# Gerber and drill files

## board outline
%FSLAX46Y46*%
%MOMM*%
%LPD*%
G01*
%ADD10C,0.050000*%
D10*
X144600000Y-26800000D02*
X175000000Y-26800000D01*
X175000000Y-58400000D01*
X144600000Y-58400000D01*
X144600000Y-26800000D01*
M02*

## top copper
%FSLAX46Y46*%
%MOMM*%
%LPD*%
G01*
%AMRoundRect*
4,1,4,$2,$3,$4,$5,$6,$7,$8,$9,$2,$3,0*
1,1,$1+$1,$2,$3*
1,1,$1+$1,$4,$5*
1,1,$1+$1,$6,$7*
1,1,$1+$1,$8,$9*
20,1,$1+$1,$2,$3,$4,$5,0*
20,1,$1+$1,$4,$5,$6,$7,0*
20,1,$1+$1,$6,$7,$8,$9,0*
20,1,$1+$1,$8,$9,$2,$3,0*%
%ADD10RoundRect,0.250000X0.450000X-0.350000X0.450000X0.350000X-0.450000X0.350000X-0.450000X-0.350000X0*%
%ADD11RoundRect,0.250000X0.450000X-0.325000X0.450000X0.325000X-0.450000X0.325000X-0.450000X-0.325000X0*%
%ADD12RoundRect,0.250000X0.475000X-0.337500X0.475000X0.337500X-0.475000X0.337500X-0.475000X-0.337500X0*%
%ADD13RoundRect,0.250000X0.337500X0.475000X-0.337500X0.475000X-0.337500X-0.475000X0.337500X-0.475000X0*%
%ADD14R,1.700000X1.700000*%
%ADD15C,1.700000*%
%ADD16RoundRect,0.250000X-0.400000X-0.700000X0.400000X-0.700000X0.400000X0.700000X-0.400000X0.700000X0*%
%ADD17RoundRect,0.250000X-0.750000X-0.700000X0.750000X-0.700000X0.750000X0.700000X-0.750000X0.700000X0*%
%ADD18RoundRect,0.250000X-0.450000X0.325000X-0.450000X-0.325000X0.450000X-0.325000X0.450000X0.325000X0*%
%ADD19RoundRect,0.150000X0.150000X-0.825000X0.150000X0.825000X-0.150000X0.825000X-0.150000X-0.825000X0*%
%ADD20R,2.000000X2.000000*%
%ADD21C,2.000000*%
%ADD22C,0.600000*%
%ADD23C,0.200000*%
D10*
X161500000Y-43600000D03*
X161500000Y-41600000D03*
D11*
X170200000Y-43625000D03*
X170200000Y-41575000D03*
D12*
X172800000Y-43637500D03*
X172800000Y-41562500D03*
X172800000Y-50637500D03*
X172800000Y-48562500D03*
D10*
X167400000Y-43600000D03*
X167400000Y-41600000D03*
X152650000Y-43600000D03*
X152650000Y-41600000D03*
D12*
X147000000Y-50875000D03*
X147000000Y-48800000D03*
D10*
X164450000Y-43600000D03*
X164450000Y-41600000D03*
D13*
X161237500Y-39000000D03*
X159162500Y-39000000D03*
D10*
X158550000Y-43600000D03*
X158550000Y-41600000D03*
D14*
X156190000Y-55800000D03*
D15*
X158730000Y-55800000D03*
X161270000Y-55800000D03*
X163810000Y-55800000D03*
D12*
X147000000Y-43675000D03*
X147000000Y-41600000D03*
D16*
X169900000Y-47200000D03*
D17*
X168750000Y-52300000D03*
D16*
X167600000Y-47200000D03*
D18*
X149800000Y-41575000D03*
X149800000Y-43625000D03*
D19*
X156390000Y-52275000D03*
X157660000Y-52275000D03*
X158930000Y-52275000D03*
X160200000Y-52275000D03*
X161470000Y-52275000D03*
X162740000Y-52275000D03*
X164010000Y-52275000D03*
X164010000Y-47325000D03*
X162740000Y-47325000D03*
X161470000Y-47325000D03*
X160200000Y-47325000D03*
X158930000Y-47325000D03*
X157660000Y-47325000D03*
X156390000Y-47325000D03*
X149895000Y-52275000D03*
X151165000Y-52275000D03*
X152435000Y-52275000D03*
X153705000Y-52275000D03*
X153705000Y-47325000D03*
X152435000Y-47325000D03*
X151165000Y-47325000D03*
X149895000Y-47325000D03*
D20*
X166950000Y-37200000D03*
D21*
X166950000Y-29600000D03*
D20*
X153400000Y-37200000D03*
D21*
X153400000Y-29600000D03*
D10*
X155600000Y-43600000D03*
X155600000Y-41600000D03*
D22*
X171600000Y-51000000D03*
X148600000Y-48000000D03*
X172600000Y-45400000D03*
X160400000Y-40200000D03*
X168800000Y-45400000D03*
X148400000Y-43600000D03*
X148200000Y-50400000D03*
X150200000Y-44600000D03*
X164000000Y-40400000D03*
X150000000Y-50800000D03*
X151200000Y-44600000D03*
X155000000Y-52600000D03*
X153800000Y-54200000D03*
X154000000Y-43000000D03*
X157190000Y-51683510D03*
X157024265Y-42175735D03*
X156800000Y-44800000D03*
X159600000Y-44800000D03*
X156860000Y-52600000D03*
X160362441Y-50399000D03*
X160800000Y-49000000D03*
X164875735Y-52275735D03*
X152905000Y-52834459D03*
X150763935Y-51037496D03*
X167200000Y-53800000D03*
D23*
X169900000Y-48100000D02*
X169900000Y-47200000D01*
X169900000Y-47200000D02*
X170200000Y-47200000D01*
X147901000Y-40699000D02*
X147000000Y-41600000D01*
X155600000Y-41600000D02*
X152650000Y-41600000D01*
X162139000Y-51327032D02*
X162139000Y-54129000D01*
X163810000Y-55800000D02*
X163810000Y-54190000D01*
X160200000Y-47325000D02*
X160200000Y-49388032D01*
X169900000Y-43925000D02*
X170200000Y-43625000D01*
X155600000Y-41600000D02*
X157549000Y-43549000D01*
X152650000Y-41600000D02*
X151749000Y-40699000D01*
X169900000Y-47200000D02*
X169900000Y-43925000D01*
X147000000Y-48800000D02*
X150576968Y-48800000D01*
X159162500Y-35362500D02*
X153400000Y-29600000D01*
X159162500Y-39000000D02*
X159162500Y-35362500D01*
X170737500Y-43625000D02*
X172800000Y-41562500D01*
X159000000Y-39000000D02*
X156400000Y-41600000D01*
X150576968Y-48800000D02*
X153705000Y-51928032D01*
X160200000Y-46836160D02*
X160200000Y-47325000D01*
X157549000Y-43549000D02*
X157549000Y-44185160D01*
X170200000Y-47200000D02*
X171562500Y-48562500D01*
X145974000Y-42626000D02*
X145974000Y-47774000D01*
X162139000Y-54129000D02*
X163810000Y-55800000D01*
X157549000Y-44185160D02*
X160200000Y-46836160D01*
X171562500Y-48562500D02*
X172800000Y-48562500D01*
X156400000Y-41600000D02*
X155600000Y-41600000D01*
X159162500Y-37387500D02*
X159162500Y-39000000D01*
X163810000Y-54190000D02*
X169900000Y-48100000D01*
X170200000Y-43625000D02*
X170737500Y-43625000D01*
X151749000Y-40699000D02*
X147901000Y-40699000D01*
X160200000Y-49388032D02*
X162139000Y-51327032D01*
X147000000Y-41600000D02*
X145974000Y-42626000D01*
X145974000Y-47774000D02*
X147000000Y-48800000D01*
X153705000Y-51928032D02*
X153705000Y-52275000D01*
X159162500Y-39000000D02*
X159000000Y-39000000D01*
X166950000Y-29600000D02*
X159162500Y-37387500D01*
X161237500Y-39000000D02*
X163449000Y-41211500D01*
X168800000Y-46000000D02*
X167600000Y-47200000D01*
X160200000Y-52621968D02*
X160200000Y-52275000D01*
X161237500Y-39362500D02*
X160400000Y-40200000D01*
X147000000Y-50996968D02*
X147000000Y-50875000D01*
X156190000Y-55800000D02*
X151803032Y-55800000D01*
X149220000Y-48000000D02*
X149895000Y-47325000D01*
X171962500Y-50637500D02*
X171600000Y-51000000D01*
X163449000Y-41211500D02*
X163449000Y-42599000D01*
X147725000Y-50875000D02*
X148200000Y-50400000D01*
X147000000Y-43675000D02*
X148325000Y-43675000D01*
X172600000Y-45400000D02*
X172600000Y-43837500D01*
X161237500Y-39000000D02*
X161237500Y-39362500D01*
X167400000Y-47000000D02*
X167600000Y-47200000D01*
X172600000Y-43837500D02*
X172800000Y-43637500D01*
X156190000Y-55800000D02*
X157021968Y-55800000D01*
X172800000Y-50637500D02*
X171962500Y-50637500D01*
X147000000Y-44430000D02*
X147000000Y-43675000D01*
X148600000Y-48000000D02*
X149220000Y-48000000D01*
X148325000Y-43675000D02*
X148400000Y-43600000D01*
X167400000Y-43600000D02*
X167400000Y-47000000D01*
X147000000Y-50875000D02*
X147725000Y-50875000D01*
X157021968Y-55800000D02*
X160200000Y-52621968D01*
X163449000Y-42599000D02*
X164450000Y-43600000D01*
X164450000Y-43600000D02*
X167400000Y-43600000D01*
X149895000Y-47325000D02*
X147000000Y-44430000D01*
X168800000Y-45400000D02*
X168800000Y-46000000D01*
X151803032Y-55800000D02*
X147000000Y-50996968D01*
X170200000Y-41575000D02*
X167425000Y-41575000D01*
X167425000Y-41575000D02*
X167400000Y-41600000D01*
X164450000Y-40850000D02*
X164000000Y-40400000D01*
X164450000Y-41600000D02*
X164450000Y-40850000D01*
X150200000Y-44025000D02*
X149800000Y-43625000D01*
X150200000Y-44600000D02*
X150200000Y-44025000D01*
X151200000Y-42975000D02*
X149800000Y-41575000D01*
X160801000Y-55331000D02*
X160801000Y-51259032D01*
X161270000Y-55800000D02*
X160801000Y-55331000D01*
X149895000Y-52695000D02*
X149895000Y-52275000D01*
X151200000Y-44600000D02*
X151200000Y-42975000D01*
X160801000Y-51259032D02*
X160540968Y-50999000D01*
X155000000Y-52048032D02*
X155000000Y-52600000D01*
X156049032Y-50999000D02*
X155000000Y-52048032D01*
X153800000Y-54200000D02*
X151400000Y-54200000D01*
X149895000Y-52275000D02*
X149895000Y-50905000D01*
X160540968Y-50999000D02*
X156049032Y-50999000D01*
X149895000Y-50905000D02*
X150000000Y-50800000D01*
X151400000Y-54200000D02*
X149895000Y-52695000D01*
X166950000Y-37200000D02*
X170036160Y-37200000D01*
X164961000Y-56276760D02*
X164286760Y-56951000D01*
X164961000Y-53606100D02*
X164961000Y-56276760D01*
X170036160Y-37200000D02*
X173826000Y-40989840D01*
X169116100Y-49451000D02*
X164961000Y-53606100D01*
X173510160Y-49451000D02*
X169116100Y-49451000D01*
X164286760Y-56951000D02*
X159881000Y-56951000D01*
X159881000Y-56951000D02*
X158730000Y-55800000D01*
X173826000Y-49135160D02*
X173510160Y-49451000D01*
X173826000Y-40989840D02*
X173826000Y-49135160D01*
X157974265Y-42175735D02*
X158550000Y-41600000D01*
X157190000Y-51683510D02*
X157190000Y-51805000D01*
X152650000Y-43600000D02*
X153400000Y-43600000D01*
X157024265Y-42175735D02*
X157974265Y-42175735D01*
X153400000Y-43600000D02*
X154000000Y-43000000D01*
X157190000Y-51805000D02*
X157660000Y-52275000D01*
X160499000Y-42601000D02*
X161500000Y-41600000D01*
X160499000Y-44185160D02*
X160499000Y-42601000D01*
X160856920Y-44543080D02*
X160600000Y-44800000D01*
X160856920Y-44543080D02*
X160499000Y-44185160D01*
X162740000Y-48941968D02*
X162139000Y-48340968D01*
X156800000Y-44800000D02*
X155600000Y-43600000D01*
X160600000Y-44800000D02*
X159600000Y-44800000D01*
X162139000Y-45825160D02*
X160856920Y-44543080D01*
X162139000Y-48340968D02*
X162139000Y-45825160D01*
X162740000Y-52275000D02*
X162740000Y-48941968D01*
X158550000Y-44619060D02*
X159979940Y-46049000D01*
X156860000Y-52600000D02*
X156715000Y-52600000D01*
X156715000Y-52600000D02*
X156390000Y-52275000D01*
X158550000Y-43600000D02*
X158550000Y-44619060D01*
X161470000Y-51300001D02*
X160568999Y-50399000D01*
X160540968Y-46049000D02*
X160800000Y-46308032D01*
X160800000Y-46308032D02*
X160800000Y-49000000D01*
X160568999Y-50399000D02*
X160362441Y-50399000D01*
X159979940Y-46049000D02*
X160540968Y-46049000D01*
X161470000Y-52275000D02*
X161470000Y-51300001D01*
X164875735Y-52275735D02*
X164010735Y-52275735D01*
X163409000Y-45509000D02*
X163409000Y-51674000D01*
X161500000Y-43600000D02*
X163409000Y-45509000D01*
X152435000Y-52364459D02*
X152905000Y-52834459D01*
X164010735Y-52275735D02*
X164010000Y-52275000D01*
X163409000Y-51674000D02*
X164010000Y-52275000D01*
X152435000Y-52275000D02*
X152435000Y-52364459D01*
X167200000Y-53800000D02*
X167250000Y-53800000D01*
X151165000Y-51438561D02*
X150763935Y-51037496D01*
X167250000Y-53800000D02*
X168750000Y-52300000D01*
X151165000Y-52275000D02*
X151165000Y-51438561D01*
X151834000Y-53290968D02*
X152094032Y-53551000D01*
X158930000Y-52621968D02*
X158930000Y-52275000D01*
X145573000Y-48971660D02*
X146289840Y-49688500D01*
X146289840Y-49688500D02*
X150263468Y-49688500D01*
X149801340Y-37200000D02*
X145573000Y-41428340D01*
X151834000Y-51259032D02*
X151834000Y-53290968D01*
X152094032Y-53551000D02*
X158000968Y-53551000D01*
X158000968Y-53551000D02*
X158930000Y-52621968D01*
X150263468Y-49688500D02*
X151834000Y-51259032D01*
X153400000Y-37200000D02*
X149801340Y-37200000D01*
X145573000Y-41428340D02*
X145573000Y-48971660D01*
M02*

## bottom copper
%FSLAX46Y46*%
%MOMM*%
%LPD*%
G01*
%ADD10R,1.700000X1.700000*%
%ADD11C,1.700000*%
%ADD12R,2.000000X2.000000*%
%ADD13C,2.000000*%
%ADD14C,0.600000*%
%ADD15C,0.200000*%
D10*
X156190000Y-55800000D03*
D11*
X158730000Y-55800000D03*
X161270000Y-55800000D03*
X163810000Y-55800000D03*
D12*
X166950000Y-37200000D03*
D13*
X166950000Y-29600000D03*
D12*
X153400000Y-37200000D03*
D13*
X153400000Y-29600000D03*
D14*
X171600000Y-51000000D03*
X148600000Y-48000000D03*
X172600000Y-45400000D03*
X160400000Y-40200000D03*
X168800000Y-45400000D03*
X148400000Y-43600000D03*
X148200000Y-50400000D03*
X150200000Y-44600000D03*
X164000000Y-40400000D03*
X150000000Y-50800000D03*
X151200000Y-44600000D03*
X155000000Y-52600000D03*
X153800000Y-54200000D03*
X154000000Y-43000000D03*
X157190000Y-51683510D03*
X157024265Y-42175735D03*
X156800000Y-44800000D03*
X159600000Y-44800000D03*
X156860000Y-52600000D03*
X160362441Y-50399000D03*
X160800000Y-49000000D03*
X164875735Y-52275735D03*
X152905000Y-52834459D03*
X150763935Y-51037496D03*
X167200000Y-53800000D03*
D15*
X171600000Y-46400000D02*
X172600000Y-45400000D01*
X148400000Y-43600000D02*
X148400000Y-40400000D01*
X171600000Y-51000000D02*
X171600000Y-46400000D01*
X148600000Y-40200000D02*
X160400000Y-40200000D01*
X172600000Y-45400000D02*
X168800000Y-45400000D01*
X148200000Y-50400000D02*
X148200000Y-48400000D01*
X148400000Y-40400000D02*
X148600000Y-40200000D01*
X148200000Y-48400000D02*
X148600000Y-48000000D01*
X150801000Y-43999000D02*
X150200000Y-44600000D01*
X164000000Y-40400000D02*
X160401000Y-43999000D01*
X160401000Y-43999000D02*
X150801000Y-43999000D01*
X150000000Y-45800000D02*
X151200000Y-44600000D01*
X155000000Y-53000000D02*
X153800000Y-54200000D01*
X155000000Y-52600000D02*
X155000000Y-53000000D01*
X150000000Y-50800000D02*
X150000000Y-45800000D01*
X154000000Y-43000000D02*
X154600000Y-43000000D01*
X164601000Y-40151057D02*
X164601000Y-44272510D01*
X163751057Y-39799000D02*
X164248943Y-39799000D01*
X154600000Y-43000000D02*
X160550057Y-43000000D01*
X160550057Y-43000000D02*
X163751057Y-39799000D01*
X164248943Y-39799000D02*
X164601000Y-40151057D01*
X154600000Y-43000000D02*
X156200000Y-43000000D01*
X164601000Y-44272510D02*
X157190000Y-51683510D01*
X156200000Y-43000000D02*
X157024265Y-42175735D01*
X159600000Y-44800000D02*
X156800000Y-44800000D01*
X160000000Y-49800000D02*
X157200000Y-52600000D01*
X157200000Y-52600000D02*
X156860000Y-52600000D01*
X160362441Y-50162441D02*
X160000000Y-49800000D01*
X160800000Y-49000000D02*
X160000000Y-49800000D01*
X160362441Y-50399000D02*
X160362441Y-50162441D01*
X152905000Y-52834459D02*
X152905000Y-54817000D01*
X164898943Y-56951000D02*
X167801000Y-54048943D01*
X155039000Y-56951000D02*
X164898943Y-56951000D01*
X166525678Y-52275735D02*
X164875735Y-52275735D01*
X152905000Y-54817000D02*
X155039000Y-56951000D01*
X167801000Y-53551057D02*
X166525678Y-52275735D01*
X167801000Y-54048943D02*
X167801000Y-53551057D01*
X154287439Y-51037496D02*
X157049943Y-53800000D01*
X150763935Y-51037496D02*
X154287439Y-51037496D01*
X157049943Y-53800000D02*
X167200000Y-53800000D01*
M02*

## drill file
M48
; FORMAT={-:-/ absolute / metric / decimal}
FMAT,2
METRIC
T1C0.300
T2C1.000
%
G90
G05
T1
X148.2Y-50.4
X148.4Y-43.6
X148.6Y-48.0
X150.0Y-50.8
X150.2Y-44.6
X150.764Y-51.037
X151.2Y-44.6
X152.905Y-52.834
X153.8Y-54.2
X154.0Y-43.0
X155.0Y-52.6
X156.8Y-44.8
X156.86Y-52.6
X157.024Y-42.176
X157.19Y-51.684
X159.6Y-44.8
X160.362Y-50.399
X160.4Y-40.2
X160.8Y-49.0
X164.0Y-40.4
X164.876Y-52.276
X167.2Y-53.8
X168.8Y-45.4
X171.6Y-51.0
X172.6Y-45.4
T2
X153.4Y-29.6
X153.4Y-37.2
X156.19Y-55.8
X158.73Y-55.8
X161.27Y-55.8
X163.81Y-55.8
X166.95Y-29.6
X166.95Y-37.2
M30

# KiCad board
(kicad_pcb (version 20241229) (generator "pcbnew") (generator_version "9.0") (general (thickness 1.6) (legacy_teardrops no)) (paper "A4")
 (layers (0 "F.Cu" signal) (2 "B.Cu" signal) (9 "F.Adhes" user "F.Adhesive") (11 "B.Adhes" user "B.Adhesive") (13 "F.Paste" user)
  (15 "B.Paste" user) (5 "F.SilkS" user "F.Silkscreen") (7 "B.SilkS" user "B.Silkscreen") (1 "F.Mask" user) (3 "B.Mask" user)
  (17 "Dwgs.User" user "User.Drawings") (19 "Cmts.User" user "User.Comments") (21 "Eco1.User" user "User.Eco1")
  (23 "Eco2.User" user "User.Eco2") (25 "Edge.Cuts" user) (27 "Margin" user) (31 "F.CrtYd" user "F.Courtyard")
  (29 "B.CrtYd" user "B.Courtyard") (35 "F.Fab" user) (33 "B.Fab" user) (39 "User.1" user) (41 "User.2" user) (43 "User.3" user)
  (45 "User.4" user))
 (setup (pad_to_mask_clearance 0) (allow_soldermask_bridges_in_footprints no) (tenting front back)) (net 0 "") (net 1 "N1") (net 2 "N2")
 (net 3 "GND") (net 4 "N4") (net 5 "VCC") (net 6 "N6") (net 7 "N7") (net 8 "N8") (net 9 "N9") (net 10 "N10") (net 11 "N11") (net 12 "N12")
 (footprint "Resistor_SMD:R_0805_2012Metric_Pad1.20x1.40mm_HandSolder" (layer "F.Cu") (at 161.5 42.6 90)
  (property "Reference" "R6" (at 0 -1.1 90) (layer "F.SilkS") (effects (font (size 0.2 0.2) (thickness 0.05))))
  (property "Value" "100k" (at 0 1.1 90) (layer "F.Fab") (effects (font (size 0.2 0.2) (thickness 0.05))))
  (pad "1" smd roundrect (at -1 0 90) (size 1.2 1.4) (layers "F.Cu" "F.Mask" "F.Paste") (roundrect_rratio 0.208333) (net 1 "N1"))
  (pad "2" smd roundrect (at 1 0 90) (size 1.2 1.4) (layers "F.Cu" "F.Mask" "F.Paste") (roundrect_rratio 0.208333) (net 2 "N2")))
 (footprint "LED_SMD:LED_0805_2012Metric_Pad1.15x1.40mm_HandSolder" (layer "F.Cu") (at 170.2 42.6 90)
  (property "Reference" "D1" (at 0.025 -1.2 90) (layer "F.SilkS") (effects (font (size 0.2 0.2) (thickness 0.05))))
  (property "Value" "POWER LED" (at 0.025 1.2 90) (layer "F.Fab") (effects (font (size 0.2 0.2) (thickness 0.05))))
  (pad "1" smd roundrect (at -1.025 0 90) (size 1.15 1.4) (layers "F.Cu" "F.Mask" "F.Paste") (roundrect_rratio 0.217391) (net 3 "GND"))
  (pad "2" smd roundrect (at 1.025 0 90) (size 1.15 1.4) (layers "F.Cu" "F.Mask" "F.Paste") (roundrect_rratio 0.217391) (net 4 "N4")))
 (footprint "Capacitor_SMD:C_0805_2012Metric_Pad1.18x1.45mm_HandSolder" (layer "F.Cu") (at 172.8 42.6 90)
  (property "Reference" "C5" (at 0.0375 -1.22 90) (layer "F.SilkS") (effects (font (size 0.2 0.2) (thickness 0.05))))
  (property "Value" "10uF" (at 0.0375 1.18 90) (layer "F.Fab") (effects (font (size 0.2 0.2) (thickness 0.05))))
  (pad "1" smd roundrect (at -1.0375 0 90) (size 1.175 1.45) (layers "F.Cu" "F.Mask" "F.Paste") (roundrect_rratio 0.212766) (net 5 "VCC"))
  (pad "2" smd roundrect (at 1.0375 0 90) (size 1.175 1.45) (layers "F.Cu" "F.Mask" "F.Paste") (roundrect_rratio 0.212766) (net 3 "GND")))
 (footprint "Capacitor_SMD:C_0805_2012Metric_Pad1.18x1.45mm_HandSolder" (layer "F.Cu") (at 172.8 49.6 90)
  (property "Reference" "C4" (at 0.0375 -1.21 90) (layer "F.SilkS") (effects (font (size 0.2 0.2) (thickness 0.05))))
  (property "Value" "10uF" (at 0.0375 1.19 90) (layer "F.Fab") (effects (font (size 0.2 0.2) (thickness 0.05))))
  (pad "1" smd roundrect (at -1.0375 0 90) (size 1.175 1.45) (layers "F.Cu" "F.Mask" "F.Paste") (roundrect_rratio 0.212766) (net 5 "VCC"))
  (pad "2" smd roundrect (at 1.0375 0 90) (size 1.175 1.45) (layers "F.Cu" "F.Mask" "F.Paste") (roundrect_rratio 0.212766) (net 3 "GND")))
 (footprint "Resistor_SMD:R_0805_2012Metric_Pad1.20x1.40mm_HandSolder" (layer "F.Cu") (at 167.4 42.6 90)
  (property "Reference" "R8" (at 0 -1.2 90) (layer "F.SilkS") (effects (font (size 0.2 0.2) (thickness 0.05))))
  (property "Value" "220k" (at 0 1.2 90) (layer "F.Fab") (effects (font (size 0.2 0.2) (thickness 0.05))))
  (pad "1" smd roundrect (at -1 0 90) (size 1.2 1.4) (layers "F.Cu" "F.Mask" "F.Paste") (roundrect_rratio 0.208333) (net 5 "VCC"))
  (pad "2" smd roundrect (at 1 0 90) (size 1.2 1.4) (layers "F.Cu" "F.Mask" "F.Paste") (roundrect_rratio 0.208333) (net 4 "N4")))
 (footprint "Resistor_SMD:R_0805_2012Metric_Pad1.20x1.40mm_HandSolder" (layer "F.Cu") (at 152.65 42.6 90)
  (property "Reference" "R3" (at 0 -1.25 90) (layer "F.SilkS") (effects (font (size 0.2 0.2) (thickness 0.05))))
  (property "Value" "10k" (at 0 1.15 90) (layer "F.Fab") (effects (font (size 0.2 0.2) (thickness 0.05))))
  (pad "1" smd roundrect (at -1 0 90) (size 1.2 1.4) (layers "F.Cu" "F.Mask" "F.Paste") (roundrect_rratio 0.208333) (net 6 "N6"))
  (pad "2" smd roundrect (at 1 0 90) (size 1.2 1.4) (layers "F.Cu" "F.Mask" "F.Paste") (roundrect_rratio 0.208333) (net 3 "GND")))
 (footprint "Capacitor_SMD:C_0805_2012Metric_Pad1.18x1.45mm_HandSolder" (layer "F.Cu") (at 147 49.8375 90)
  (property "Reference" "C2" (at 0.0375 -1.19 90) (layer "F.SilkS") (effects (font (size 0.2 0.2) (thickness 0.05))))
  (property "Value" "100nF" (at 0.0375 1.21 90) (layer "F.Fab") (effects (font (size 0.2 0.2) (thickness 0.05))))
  (pad "1" smd roundrect (at -1.0375 0 90) (size 1.175 1.45) (layers "F.Cu" "F.Mask" "F.Paste") (roundrect_rratio 0.212766) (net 5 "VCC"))
  (pad "2" smd roundrect (at 1.0375 0 90) (size 1.175 1.45) (layers "F.Cu" "F.Mask" "F.Paste") (roundrect_rratio 0.212766) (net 3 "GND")))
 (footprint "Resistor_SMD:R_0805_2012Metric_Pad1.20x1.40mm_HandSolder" (layer "F.Cu") (at 164.45 42.6 90)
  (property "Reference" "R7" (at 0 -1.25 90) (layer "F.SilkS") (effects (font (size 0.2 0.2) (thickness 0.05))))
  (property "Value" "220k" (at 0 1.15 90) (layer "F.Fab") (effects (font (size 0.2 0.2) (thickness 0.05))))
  (pad "1" smd roundrect (at -1 0 90) (size 1.2 1.4) (layers "F.Cu" "F.Mask" "F.Paste") (roundrect_rratio 0.208333) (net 5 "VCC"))
  (pad "2" smd roundrect (at 1 0 90) (size 1.2 1.4) (layers "F.Cu" "F.Mask" "F.Paste") (roundrect_rratio 0.208333) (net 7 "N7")))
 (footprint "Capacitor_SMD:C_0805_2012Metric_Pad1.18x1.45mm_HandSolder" (layer "F.Cu") (at 160.2 39 180)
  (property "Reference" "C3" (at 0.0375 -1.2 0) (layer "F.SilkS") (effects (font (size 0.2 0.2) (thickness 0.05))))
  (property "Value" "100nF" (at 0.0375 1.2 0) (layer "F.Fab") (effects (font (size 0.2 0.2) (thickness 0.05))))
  (pad "1" smd roundrect (at -1.0375 0 180) (size 1.175 1.45) (layers "F.Cu" "F.Mask" "F.Paste") (roundrect_rratio 0.212766) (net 5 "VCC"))
  (pad "2" smd roundrect (at 1.0375 0 180) (size 1.175 1.45) (layers "F.Cu" "F.Mask" "F.Paste") (roundrect_rratio 0.212766) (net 3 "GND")))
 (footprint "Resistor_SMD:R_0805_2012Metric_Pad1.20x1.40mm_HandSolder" (layer "F.Cu") (at 158.55 42.6 90)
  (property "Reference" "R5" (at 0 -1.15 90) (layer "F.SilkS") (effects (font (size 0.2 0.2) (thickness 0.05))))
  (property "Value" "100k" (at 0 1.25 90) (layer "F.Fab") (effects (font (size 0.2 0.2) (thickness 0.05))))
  (pad "1" smd roundrect (at -1 0 90) (size 1.2 1.4) (layers "F.Cu" "F.Mask" "F.Paste") (roundrect_rratio 0.208333) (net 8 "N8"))
  (pad "2" smd roundrect (at 1 0 90) (size 1.2 1.4) (layers "F.Cu" "F.Mask" "F.Paste") (roundrect_rratio 0.208333) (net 6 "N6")))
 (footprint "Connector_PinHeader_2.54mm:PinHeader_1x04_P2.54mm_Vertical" (layer "F.Cu") (at 156.19 55.8 90)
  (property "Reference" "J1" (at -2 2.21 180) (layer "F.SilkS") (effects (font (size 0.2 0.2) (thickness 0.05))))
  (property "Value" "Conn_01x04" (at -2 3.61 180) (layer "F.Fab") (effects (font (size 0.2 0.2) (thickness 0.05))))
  (pad "1" thru_hole rect (at 0 0 90) (size 1.7 1.7) (drill 1) (layers "*.Cu" "*.Mask") (remove_unused_layers no) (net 5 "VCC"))
  (pad "2" thru_hole circle (at 0 2.54 90) (size 1.7 1.7) (drill 1) (layers "*.Cu" "*.Mask") (remove_unused_layers no) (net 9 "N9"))
  (pad "3" thru_hole circle (at 0 5.08 90) (size 1.7 1.7) (drill 1) (layers "*.Cu" "*.Mask") (remove_unused_layers no) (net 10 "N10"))
  (pad "4" thru_hole circle (at 0 7.62 90) (size 1.7 1.7) (drill 1) (layers "*.Cu" "*.Mask") (remove_unused_layers no) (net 3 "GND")))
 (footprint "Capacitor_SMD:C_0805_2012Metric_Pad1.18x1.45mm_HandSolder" (layer "F.Cu") (at 147 42.6375 90)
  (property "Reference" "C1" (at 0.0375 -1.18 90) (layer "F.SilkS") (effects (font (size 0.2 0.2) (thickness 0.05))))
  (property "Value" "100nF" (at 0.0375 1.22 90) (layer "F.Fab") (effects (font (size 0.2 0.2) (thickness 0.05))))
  (pad "1" smd roundrect (at -1.0375 0 90) (size 1.175 1.45) (layers "F.Cu" "F.Mask" "F.Paste") (roundrect_rratio 0.212766) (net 5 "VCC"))
  (pad "2" smd roundrect (at 1.0375 0 90) (size 1.175 1.45) (layers "F.Cu" "F.Mask" "F.Paste") (roundrect_rratio 0.212766) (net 3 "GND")))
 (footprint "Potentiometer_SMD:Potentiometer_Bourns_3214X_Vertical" (layer "F.Cu") (at 168.75 49.75)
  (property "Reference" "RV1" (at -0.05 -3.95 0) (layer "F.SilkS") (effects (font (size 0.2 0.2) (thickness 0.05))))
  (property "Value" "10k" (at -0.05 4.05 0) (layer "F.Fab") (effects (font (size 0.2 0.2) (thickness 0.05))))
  (pad "1" smd roundrect (at 1.15 -2.55) (size 1.3 1.9) (layers "F.Cu" "F.Mask" "F.Paste") (roundrect_rratio 0.192308) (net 3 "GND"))
  (pad "2" smd roundrect (at 0 2.55) (size 2 1.9) (layers "F.Cu" "F.Mask" "F.Paste") (roundrect_rratio 0.131579) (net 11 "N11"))
  (pad "3" smd roundrect (at -1.15 -2.55) (size 1.3 1.9) (layers "F.Cu" "F.Mask" "F.Paste") (roundrect_rratio 0.192308) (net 5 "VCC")))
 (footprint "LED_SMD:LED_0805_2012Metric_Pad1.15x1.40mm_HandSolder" (layer "F.Cu") (at 149.8 42.6 -90)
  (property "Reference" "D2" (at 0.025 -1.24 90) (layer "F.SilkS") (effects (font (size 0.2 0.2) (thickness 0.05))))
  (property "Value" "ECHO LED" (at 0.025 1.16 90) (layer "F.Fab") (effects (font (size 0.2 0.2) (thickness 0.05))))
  (pad "1" smd roundrect (at -1.025 0 270) (size 1.15 1.4) (layers "F.Cu" "F.Mask" "F.Paste") (roundrect_rratio 0.217391) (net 10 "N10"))
  (pad "2" smd roundrect (at 1.025 0 270) (size 1.15 1.4) (layers "F.Cu" "F.Mask" "F.Paste") (roundrect_rratio 0.217391) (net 7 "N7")))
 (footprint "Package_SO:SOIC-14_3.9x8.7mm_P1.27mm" (layer "F.Cu") (at 160.2 49.8 90)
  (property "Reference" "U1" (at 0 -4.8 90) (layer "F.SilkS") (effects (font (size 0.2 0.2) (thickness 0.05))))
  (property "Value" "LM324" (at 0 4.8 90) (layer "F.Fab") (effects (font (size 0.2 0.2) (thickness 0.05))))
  (pad "1" smd roundrect (at -2.475 -3.81 90) (size 1.95 0.6) (layers "F.Cu" "F.Mask" "F.Paste") (roundrect_rratio 0.25) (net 8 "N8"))
  (pad "2" smd roundrect (at -2.475 -2.54 90) (size 1.95 0.6) (layers "F.Cu" "F.Mask" "F.Paste") (roundrect_rratio 0.25) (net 6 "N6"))
  (pad "3" smd roundrect (at -2.475 -1.27 90) (size 1.95 0.6) (layers "F.Cu" "F.Mask" "F.Paste") (roundrect_rratio 0.25) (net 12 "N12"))
  (pad "4" smd roundrect (at -2.475 0 90) (size 1.95 0.6) (layers "F.Cu" "F.Mask" "F.Paste") (roundrect_rratio 0.25) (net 5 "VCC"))
  (pad "5" smd roundrect (at -2.475 1.27 90) (size 1.95 0.6) (layers "F.Cu" "F.Mask" "F.Paste") (roundrect_rratio 0.25) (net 8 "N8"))
  (pad "6" smd roundrect (at -2.475 2.54 90) (size 1.95 0.6) (layers "F.Cu" "F.Mask" "F.Paste") (roundrect_rratio 0.25) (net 2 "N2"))
  (pad "7" smd roundrect (at -2.475 3.81 90) (size 1.95 0.6) (layers "F.Cu" "F.Mask" "F.Paste") (roundrect_rratio 0.25) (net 1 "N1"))
  (pad "8" smd roundrect (at 2.475 3.81 90) (size 1.95 0.6) (layers "F.Cu" "F.Mask" "F.Paste") (roundrect_rratio 0.25))
  (pad "9" smd roundrect (at 2.475 2.54 90) (size 1.95 0.6) (layers "F.Cu" "F.Mask" "F.Paste") (roundrect_rratio 0.25))
  (pad "10" smd roundrect (at 2.475 1.27 90) (size 1.95 0.6) (layers "F.Cu" "F.Mask" "F.Paste") (roundrect_rratio 0.25))
  (pad "11" smd roundrect (at 2.475 0 90) (size 1.95 0.6) (layers "F.Cu" "F.Mask" "F.Paste") (roundrect_rratio 0.25) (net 3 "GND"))
  (pad "12" smd roundrect (at 2.475 -1.27 90) (size 1.95 0.6) (layers "F.Cu" "F.Mask" "F.Paste") (roundrect_rratio 0.25))
  (pad "13" smd roundrect (at 2.475 -2.54 90) (size 1.95 0.6) (layers "F.Cu" "F.Mask" "F.Paste") (roundrect_rratio 0.25))
  (pad "14" smd roundrect (at 2.475 -3.81 90) (size 1.95 0.6) (layers "F.Cu" "F.Mask" "F.Paste") (roundrect_rratio 0.25)))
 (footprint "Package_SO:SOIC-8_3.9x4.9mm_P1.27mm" (layer "F.Cu") (at 151.8 49.8 90)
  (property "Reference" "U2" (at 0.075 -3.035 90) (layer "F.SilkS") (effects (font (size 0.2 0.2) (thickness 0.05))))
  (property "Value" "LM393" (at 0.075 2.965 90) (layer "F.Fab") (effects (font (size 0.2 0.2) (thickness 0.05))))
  (pad "1" smd roundrect (at -2.475 -1.905 90) (size 1.95 0.6) (layers "F.Cu" "F.Mask" "F.Paste") (roundrect_rratio 0.25) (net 10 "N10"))
  (pad "2" smd roundrect (at -2.475 -0.635 90) (size 1.95 0.6) (layers "F.Cu" "F.Mask" "F.Paste") (roundrect_rratio 0.25) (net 11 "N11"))
  (pad "3" smd roundrect (at -2.475 0.635 90) (size 1.95 0.6) (layers "F.Cu" "F.Mask" "F.Paste") (roundrect_rratio 0.25) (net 1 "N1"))
  (pad "4" smd roundrect (at -2.475 1.905 90) (size 1.95 0.6) (layers "F.Cu" "F.Mask" "F.Paste") (roundrect_rratio 0.25) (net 3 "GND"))
  (pad "5" smd roundrect (at 2.475 1.905 90) (size 1.95 0.6) (layers "F.Cu" "F.Mask" "F.Paste") (roundrect_rratio 0.25))
  (pad "6" smd roundrect (at 2.475 0.635 90) (size 1.95 0.6) (layers "F.Cu" "F.Mask" "F.Paste") (roundrect_rratio 0.25))
  (pad "7" smd roundrect (at 2.475 -0.635 90) (size 1.95 0.6) (layers "F.Cu" "F.Mask" "F.Paste") (roundrect_rratio 0.25))
  (pad "8" smd roundrect (at 2.475 -1.905 90) (size 1.95 0.6) (layers "F.Cu" "F.Mask" "F.Paste") (roundrect_rratio 0.25) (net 5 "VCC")))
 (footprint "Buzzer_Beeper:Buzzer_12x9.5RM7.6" (layer "F.Cu") (at 166.95 37.2 90)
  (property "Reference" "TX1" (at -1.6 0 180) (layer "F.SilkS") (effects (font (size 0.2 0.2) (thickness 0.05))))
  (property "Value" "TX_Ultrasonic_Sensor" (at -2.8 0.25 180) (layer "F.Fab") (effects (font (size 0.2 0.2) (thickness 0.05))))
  (pad "1" thru_hole rect (at 0 0 90) (size 2 2) (drill 1) (layers "*.Cu" "*.Mask") (remove_unused_layers no) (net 9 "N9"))
  (pad "2" thru_hole circle (at 7.6 0 90) (size 2 2) (drill 1) (layers "*.Cu" "*.Mask") (remove_unused_layers no) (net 3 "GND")))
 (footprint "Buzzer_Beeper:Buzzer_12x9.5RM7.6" (layer "F.Cu") (at 153.4 37.2 90)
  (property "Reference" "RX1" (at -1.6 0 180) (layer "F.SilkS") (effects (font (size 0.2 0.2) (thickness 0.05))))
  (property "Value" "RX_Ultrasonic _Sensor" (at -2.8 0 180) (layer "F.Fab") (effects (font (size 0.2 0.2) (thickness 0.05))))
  (pad "1" thru_hole rect (at 0 0 90) (size 2 2) (drill 1) (layers "*.Cu" "*.Mask") (remove_unused_layers no) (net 12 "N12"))
  (pad "2" thru_hole circle (at 7.6 0 90) (size 2 2) (drill 1) (layers "*.Cu" "*.Mask") (remove_unused_layers no) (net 3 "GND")))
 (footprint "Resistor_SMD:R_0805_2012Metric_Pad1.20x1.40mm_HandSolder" (layer "F.Cu") (at 155.6 42.6 90)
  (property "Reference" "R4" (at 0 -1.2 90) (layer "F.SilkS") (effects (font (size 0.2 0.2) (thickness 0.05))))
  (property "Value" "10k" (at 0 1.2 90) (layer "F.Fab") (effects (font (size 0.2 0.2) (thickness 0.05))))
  (pad "1" smd roundrect (at -1 0 90) (size 1.2 1.4) (layers "F.Cu" "F.Mask" "F.Paste") (roundrect_rratio 0.208333) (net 2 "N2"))
  (pad "2" smd roundrect (at 1 0 90) (size 1.2 1.4) (layers "F.Cu" "F.Mask" "F.Paste") (roundrect_rratio 0.208333) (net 3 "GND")))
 (gr_rect (start 144.6 26.8) (end 175 58.4) (stroke (width 0.05) (type default)) (fill no) (layer "Edge.Cuts"))
 (segment (start 169.9 48.1) (end 169.9 47.2) (width 0.2) (layer "F.Cu") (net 3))
 (segment (start 169.9 47.2) (end 170.2 47.2) (width 0.2) (layer "F.Cu") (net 3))
 (segment (start 147.901 40.699) (end 147 41.6) (width 0.2) (layer "F.Cu") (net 3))
 (segment (start 155.6 41.6) (end 152.65 41.6) (width 0.2) (layer "F.Cu") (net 3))
 (segment (start 162.139 51.327032) (end 162.139 54.129) (width 0.2) (layer "F.Cu") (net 3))
 (segment (start 163.81 55.8) (end 163.81 54.19) (width 0.2) (layer "F.Cu") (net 3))
 (segment (start 160.2 47.325) (end 160.2 49.388032) (width 0.2) (layer "F.Cu") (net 3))
 (segment (start 169.9 43.925) (end 170.2 43.625) (width 0.2) (layer "F.Cu") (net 3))
 (segment (start 155.6 41.6) (end 157.549 43.549) (width 0.2) (layer "F.Cu") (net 3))
 (segment (start 152.65 41.6) (end 151.749 40.699) (width 0.2) (layer "F.Cu") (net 3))
 (segment (start 169.9 47.2) (end 169.9 43.925) (width 0.2) (layer "F.Cu") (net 3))
 (segment (start 147 48.8) (end 150.576968 48.8) (width 0.2) (layer "F.Cu") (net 3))
 (segment (start 159.1625 35.3625) (end 153.4 29.6) (width 0.2) (layer "F.Cu") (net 3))
 (segment (start 159.1625 39) (end 159.1625 35.3625) (width 0.2) (layer "F.Cu") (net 3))
 (segment (start 170.7375 43.625) (end 172.8 41.5625) (width 0.2) (layer "F.Cu") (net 3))
 (segment (start 159 39) (end 156.4 41.6) (width 0.2) (layer "F.Cu") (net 3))
 (segment (start 150.576968 48.8) (end 153.705 51.928032) (width 0.2) (layer "F.Cu") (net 3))
 (segment (start 160.2 46.83616) (end 160.2 47.325) (width 0.2) (layer "F.Cu") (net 3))
 (segment (start 157.549 43.549) (end 157.549 44.18516) (width 0.2) (layer "F.Cu") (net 3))
 (segment (start 170.2 47.2) (end 171.5625 48.5625) (width 0.2) (layer "F.Cu") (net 3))
 (segment (start 145.974 42.626) (end 145.974 47.774) (width 0.2) (layer "F.Cu") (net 3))
 (segment (start 162.139 54.129) (end 163.81 55.8) (width 0.2) (layer "F.Cu") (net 3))
 (segment (start 157.549 44.18516) (end 160.2 46.83616) (width 0.2) (layer "F.Cu") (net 3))
 (segment (start 171.5625 48.5625) (end 172.8 48.5625) (width 0.2) (layer "F.Cu") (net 3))
 (segment (start 156.4 41.6) (end 155.6 41.6) (width 0.2) (layer "F.Cu") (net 3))
 (segment (start 159.1625 37.3875) (end 159.1625 39) (width 0.2) (layer "F.Cu") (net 3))
 (segment (start 163.81 54.19) (end 169.9 48.1) (width 0.2) (layer "F.Cu") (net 3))
 (segment (start 170.2 43.625) (end 170.7375 43.625) (width 0.2) (layer "F.Cu") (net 3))
 (segment (start 151.749 40.699) (end 147.901 40.699) (width 0.2) (layer "F.Cu") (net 3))
 (segment (start 160.2 49.388032) (end 162.139 51.327032) (width 0.2) (layer "F.Cu") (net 3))
 (segment (start 147 41.6) (end 145.974 42.626) (width 0.2) (layer "F.Cu") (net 3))
 (segment (start 145.974 47.774) (end 147 48.8) (width 0.2) (layer "F.Cu") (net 3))
 (segment (start 153.705 51.928032) (end 153.705 52.275) (width 0.2) (layer "F.Cu") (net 3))
 (segment (start 159.1625 39) (end 159 39) (width 0.2) (layer "F.Cu") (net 3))
 (segment (start 166.95 29.6) (end 159.1625 37.3875) (width 0.2) (layer "F.Cu") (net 3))
 (segment (start 161.2375 39) (end 163.449 41.2115) (width 0.2) (layer "F.Cu") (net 5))
 (segment (start 168.8 46) (end 167.6 47.2) (width 0.2) (layer "F.Cu") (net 5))
 (segment (start 160.2 52.621968) (end 160.2 52.275) (width 0.2) (layer "F.Cu") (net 5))
 (segment (start 161.2375 39.3625) (end 160.4 40.2) (width 0.2) (layer "F.Cu") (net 5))
 (segment (start 147 50.996968) (end 147 50.875) (width 0.2) (layer "F.Cu") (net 5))
 (segment (start 156.19 55.8) (end 151.803032 55.8) (width 0.2) (layer "F.Cu") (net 5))
 (segment (start 149.22 48) (end 149.895 47.325) (width 0.2) (layer "F.Cu") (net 5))
 (segment (start 171.9625 50.6375) (end 171.6 51) (width 0.2) (layer "F.Cu") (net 5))
 (segment (start 163.449 41.2115) (end 163.449 42.599) (width 0.2) (layer "F.Cu") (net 5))
 (segment (start 147.725 50.875) (end 148.2 50.4) (width 0.2) (layer "F.Cu") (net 5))
 (segment (start 147 43.675) (end 148.325 43.675) (width 0.2) (layer "F.Cu") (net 5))
 (segment (start 172.6 45.4) (end 172.6 43.8375) (width 0.2) (layer "F.Cu") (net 5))
 (segment (start 161.2375 39) (end 161.2375 39.3625) (width 0.2) (layer "F.Cu") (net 5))
 (segment (start 167.4 47) (end 167.6 47.2) (width 0.2) (layer "F.Cu") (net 5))
 (segment (start 172.6 43.8375) (end 172.8 43.6375) (width 0.2) (layer "F.Cu") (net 5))
 (segment (start 156.19 55.8) (end 157.021968 55.8) (width 0.2) (layer "F.Cu") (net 5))
 (segment (start 172.8 50.6375) (end 171.9625 50.6375) (width 0.2) (layer "F.Cu") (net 5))
 (segment (start 147 44.43) (end 147 43.675) (width 0.2) (layer "F.Cu") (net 5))
 (segment (start 148.6 48) (end 149.22 48) (width 0.2) (layer "F.Cu") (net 5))
 (segment (start 148.325 43.675) (end 148.4 43.6) (width 0.2) (layer "F.Cu") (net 5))
 (segment (start 167.4 43.6) (end 167.4 47) (width 0.2) (layer "F.Cu") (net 5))
 (segment (start 147 50.875) (end 147.725 50.875) (width 0.2) (layer "F.Cu") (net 5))
 (segment (start 157.021968 55.8) (end 160.2 52.621968) (width 0.2) (layer "F.Cu") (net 5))
 (segment (start 163.449 42.599) (end 164.45 43.6) (width 0.2) (layer "F.Cu") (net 5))
 (segment (start 164.45 43.6) (end 167.4 43.6) (width 0.2) (layer "F.Cu") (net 5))
 (segment (start 149.895 47.325) (end 147 44.43) (width 0.2) (layer "F.Cu") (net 5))
 (segment (start 168.8 45.4) (end 168.8 46) (width 0.2) (layer "F.Cu") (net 5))
 (segment (start 151.803032 55.8) (end 147 50.996968) (width 0.2) (layer "F.Cu") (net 5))
 (via (at 171.6 51) (size 0.6) (drill 0.3) (layers "F.Cu" "B.Cu") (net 5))
 (via (at 148.6 48) (size 0.6) (drill 0.3) (layers "F.Cu" "B.Cu") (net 5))
 (via (at 172.6 45.4) (size 0.6) (drill 0.3) (layers "F.Cu" "B.Cu") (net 5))
 (via (at 160.4 40.2) (size 0.6) (drill 0.3) (layers "F.Cu" "B.Cu") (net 5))
 (via (at 168.8 45.4) (size 0.6) (drill 0.3) (layers "F.Cu" "B.Cu") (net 5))
 (via (at 148.4 43.6) (size 0.6) (drill 0.3) (layers "F.Cu" "B.Cu") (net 5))
 (via (at 148.2 50.4) (size 0.6) (drill 0.3) (layers "F.Cu" "B.Cu") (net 5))
 (segment (start 171.6 46.4) (end 172.6 45.4) (width 0.2) (layer "B.Cu") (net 5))
 (segment (start 148.4 43.6) (end 148.4 40.4) (width 0.2) (layer "B.Cu") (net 5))
 (segment (start 171.6 51) (end 171.6 46.4) (width 0.2) (layer "B.Cu") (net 5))
 (segment (start 148.6 40.2) (end 160.4 40.2) (width 0.2) (layer "B.Cu") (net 5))
 (segment (start 172.6 45.4) (end 168.8 45.4) (width 0.2) (layer "B.Cu") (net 5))
 (segment (start 148.2 50.4) (end 148.2 48.4) (width 0.2) (layer "B.Cu") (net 5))
 (segment (start 148.4 40.4) (end 148.6 40.2) (width 0.2) (layer "B.Cu") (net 5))
 (segment (start 148.2 48.4) (end 148.6 48) (width 0.2) (layer "B.Cu") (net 5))
 (segment (start 170.2 41.575) (end 167.425 41.575) (width 0.2) (layer "F.Cu") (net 4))
 (segment (start 167.425 41.575) (end 167.4 41.6) (width 0.2) (layer "F.Cu") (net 4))
 (segment (start 164.45 40.85) (end 164 40.4) (width 0.2) (layer "F.Cu") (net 7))
 (segment (start 164.45 41.6) (end 164.45 40.85) (width 0.2) (layer "F.Cu") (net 7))
 (segment (start 150.2 44.025) (end 149.8 43.625) (width 0.2) (layer "F.Cu") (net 7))
 (segment (start 150.2 44.6) (end 150.2 44.025) (width 0.2) (layer "F.Cu") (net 7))
 (via (at 150.2 44.6) (size 0.6) (drill 0.3) (layers "F.Cu" "B.Cu") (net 7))
 (via (at 164 40.4) (size 0.6) (drill 0.3) (layers "F.Cu" "B.Cu") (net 7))
 (segment (start 150.801 43.999) (end 150.2 44.6) (width 0.2) (layer "B.Cu") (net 7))
 (segment (start 164 40.4) (end 160.401 43.999) (width 0.2) (layer "B.Cu") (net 7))
 (segment (start 160.401 43.999) (end 150.801 43.999) (width 0.2) (layer "B.Cu") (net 7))
 (segment (start 151.2 42.975) (end 149.8 41.575) (width 0.2) (layer "F.Cu") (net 10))
 (segment (start 160.801 55.331) (end 160.801 51.259032) (width 0.2) (layer "F.Cu") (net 10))
 (segment (start 161.27 55.8) (end 160.801 55.331) (width 0.2) (layer "F.Cu") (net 10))
 (segment (start 149.895 52.695) (end 149.895 52.275) (width 0.2) (layer "F.Cu") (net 10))
 (segment (start 151.2 44.6) (end 151.2 42.975) (width 0.2) (layer "F.Cu") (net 10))
 (segment (start 160.801 51.259032) (end 160.540968 50.999) (width 0.2) (layer "F.Cu") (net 10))
 (segment (start 155 52.048032) (end 155 52.6) (width 0.2) (layer "F.Cu") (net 10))
 (segment (start 156.049032 50.999) (end 155 52.048032) (width 0.2) (layer "F.Cu") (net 10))
 (segment (start 153.8 54.2) (end 151.4 54.2) (width 0.2) (layer "F.Cu") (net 10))
 (segment (start 149.895 52.275) (end 149.895 50.905) (width 0.2) (layer "F.Cu") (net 10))
 (segment (start 160.540968 50.999) (end 156.049032 50.999) (width 0.2) (layer "F.Cu") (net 10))
 (segment (start 149.895 50.905) (end 150 50.8) (width 0.2) (layer "F.Cu") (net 10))
 (segment (start 151.4 54.2) (end 149.895 52.695) (width 0.2) (layer "F.Cu") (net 10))
 (via (at 150 50.8) (size 0.6) (drill 0.3) (layers "F.Cu" "B.Cu") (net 10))
 (via (at 151.2 44.6) (size 0.6) (drill 0.3) (layers "F.Cu" "B.Cu") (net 10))
 (via (at 155 52.6) (size 0.6) (drill 0.3) (layers "F.Cu" "B.Cu") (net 10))
 (via (at 153.8 54.2) (size 0.6) (drill 0.3) (layers "F.Cu" "B.Cu") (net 10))
 (segment (start 150 45.8) (end 151.2 44.6) (width 0.2) (layer "B.Cu") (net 10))
 (segment (start 155 53) (end 153.8 54.2) (width 0.2) (layer "B.Cu") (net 10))
 (segment (start 155 52.6) (end 155 53) (width 0.2) (layer "B.Cu") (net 10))
 (segment (start 150 50.8) (end 150 45.8) (width 0.2) (layer "B.Cu") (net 10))
 (segment (start 166.95 37.2) (end 170.03616 37.2) (width 0.2) (layer "F.Cu") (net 9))
 (segment (start 164.961 56.27676) (end 164.28676 56.951) (width 0.2) (layer "F.Cu") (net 9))
 (segment (start 164.961 53.6061) (end 164.961 56.27676) (width 0.2) (layer "F.Cu") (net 9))
 (segment (start 170.03616 37.2) (end 173.826 40.98984) (width 0.2) (layer "F.Cu") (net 9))
 (segment (start 169.1161 49.451) (end 164.961 53.6061) (width 0.2) (layer "F.Cu") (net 9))
 (segment (start 173.51016 49.451) (end 169.1161 49.451) (width 0.2) (layer "F.Cu") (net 9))
 (segment (start 164.28676 56.951) (end 159.881 56.951) (width 0.2) (layer "F.Cu") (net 9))
 (segment (start 159.881 56.951) (end 158.73 55.8) (width 0.2) (layer "F.Cu") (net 9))
 (segment (start 173.826 49.13516) (end 173.51016 49.451) (width 0.2) (layer "F.Cu") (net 9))
 (segment (start 173.826 40.98984) (end 173.826 49.13516) (width 0.2) (layer "F.Cu") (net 9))
 (segment (start 157.974265 42.175735) (end 158.55 41.6) (width 0.2) (layer "F.Cu") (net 6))
 (segment (start 157.19 51.68351) (end 157.19 51.805) (width 0.2) (layer "F.Cu") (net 6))
 (segment (start 152.65 43.6) (end 153.4 43.6) (width 0.2) (layer "F.Cu") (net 6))
 (segment (start 157.024265 42.175735) (end 157.974265 42.175735) (width 0.2) (layer "F.Cu") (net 6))
 (segment (start 153.4 43.6) (end 154 43) (width 0.2) (layer "F.Cu") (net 6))
 (segment (start 157.19 51.805) (end 157.66 52.275) (width 0.2) (layer "F.Cu") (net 6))
 (via (at 154 43) (size 0.6) (drill 0.3) (layers "F.Cu" "B.Cu") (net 6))
 (via (at 157.19 51.68351) (size 0.6) (drill 0.3) (layers "F.Cu" "B.Cu") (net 6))
 (via (at 157.024265 42.175735) (size 0.6) (drill 0.3) (layers "F.Cu" "B.Cu") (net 6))
 (segment (start 154 43) (end 154.6 43) (width 0.2) (layer "B.Cu") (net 6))
 (segment (start 164.601 40.151057) (end 164.601 44.27251) (width 0.2) (layer "B.Cu") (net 6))
 (segment (start 163.751057 39.799) (end 164.248943 39.799) (width 0.2) (layer "B.Cu") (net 6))
 (segment (start 154.6 43) (end 160.550057 43) (width 0.2) (layer "B.Cu") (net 6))
 (segment (start 160.550057 43) (end 163.751057 39.799) (width 0.2) (layer "B.Cu") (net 6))
 (segment (start 164.248943 39.799) (end 164.601 40.151057) (width 0.2) (layer "B.Cu") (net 6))
 (segment (start 154.6 43) (end 156.2 43) (width 0.2) (layer "B.Cu") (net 6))
 (segment (start 164.601 44.27251) (end 157.19 51.68351) (width 0.2) (layer "B.Cu") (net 6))
 (segment (start 156.2 43) (end 157.024265 42.175735) (width 0.2) (layer "B.Cu") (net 6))
 (segment (start 160.499 42.601) (end 161.5 41.6) (width 0.2) (layer "F.Cu") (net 2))
 (segment (start 160.499 44.18516) (end 160.499 42.601) (width 0.2) (layer "F.Cu") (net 2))
 (segment (start 160.85692 44.54308) (end 160.6 44.8) (width 0.2) (layer "F.Cu") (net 2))
 (segment (start 160.85692 44.54308) (end 160.499 44.18516) (width 0.2) (layer "F.Cu") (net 2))
 (segment (start 162.74 48.941968) (end 162.139 48.340968) (width 0.2) (layer "F.Cu") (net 2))
 (segment (start 156.8 44.8) (end 155.6 43.6) (width 0.2) (layer "F.Cu") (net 2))
 (segment (start 160.6 44.8) (end 159.6 44.8) (width 0.2) (layer "F.Cu") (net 2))
 (segment (start 162.139 45.82516) (end 160.85692 44.54308) (width 0.2) (layer "F.Cu") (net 2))
 (segment (start 162.139 48.340968) (end 162.139 45.82516) (width 0.2) (layer "F.Cu") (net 2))
 (segment (start 162.74 52.275) (end 162.74 48.941968) (width 0.2) (layer "F.Cu") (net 2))
 (via (at 156.8 44.8) (size 0.6) (drill 0.3) (layers "F.Cu" "B.Cu") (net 2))
 (via (at 159.6 44.8) (size 0.6) (drill 0.3) (layers "F.Cu" "B.Cu") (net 2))
 (segment (start 159.6 44.8) (end 156.8 44.8) (width 0.2) (layer "B.Cu") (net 2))
 (segment (start 158.55 44.61906) (end 159.97994 46.049) (width 0.2) (layer "F.Cu") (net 8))
 (segment (start 156.86 52.6) (end 156.715 52.6) (width 0.2) (layer "F.Cu") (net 8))
 (segment (start 156.715 52.6) (end 156.39 52.275) (width 0.2) (layer "F.Cu") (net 8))
 (segment (start 158.55 43.6) (end 158.55 44.61906) (width 0.2) (layer "F.Cu") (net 8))
 (segment (start 161.47 51.300001) (end 160.568999 50.399) (width 0.2) (layer "F.Cu") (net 8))
 (segment (start 160.540968 46.049) (end 160.8 46.308032) (width 0.2) (layer "F.Cu") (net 8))
 (segment (start 160.8 46.308032) (end 160.8 49) (width 0.2) (layer "F.Cu") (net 8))
 (segment (start 160.568999 50.399) (end 160.362441 50.399) (width 0.2) (layer "F.Cu") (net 8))
 (segment (start 159.97994 46.049) (end 160.540968 46.049) (width 0.2) (layer "F.Cu") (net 8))
 (segment (start 161.47 52.275) (end 161.47 51.300001) (width 0.2) (layer "F.Cu") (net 8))
 (via (at 156.86 52.6) (size 0.6) (drill 0.3) (layers "F.Cu" "B.Cu") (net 8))
 (via (at 160.362441 50.399) (size 0.6) (drill 0.3) (layers "F.Cu" "B.Cu") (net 8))
 (via (at 160.8 49) (size 0.6) (drill 0.3) (layers "F.Cu" "B.Cu") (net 8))
 (segment (start 160 49.8) (end 157.2 52.6) (width 0.2) (layer "B.Cu") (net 8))
 (segment (start 157.2 52.6) (end 156.86 52.6) (width 0.2) (layer "B.Cu") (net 8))
 (segment (start 160.362441 50.162441) (end 160 49.8) (width 0.2) (layer "B.Cu") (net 8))
 (segment (start 160.8 49) (end 160 49.8) (width 0.2) (layer "B.Cu") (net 8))
 (segment (start 160.362441 50.399) (end 160.362441 50.162441) (width 0.2) (layer "B.Cu") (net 8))
 (segment (start 164.875735 52.275735) (end 164.010735 52.275735) (width 0.2) (layer "F.Cu") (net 1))
 (segment (start 163.409 45.509) (end 163.409 51.674) (width 0.2) (layer "F.Cu") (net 1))
 (segment (start 161.5 43.6) (end 163.409 45.509) (width 0.2) (layer "F.Cu") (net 1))
 (segment (start 152.435 52.364459) (end 152.905 52.834459) (width 0.2) (layer "F.Cu") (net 1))
 (segment (start 164.010735 52.275735) (end 164.01 52.275) (width 0.2) (layer "F.Cu") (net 1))
 (segment (start 163.409 51.674) (end 164.01 52.275) (width 0.2) (layer "F.Cu") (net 1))
 (segment (start 152.435 52.275) (end 152.435 52.364459) (width 0.2) (layer "F.Cu") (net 1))
 (via (at 164.875735 52.275735) (size 0.6) (drill 0.3) (layers "F.Cu" "B.Cu") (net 1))
 (via (at 152.905 52.834459) (size 0.6) (drill 0.3) (layers "F.Cu" "B.Cu") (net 1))
 (segment (start 152.905 52.834459) (end 152.905 54.817) (width 0.2) (layer "B.Cu") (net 1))
 (segment (start 164.898943 56.951) (end 167.801 54.048943) (width 0.2) (layer "B.Cu") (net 1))
 (segment (start 155.039 56.951) (end 164.898943 56.951) (width 0.2) (layer "B.Cu") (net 1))
 (segment (start 166.525678 52.275735) (end 164.875735 52.275735) (width 0.2) (layer "B.Cu") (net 1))
 (segment (start 152.905 54.817) (end 155.039 56.951) (width 0.2) (layer "B.Cu") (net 1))
 (segment (start 167.801 53.551057) (end 166.525678 52.275735) (width 0.2) (layer "B.Cu") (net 1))
 (segment (start 167.801 54.048943) (end 167.801 53.551057) (width 0.2) (layer "B.Cu") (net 1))
 (segment (start 167.2 53.8) (end 167.25 53.8) (width 0.2) (layer "F.Cu") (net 11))
 (segment (start 151.165 51.438561) (end 150.763935 51.037496) (width 0.2) (layer "F.Cu") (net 11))
 (segment (start 167.25 53.8) (end 168.75 52.3) (width 0.2) (layer "F.Cu") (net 11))
 (segment (start 151.165 52.275) (end 151.165 51.438561) (width 0.2) (layer "F.Cu") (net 11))
 (via (at 150.763935 51.037496) (size 0.6) (drill 0.3) (layers "F.Cu" "B.Cu") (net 11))
 (via (at 167.2 53.8) (size 0.6) (drill 0.3) (layers "F.Cu" "B.Cu") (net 11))
 (segment (start 154.287439 51.037496) (end 157.049943 53.8) (width 0.2) (layer "B.Cu") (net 11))
 (segment (start 150.763935 51.037496) (end 154.287439 51.037496) (width 0.2) (layer "B.Cu") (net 11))
 (segment (start 157.049943 53.8) (end 167.2 53.8) (width 0.2) (layer "B.Cu") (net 11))
 (segment (start 151.834 53.290968) (end 152.094032 53.551) (width 0.2) (layer "F.Cu") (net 12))
 (segment (start 158.93 52.621968) (end 158.93 52.275) (width 0.2) (layer "F.Cu") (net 12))
 (segment (start 145.573 48.97166) (end 146.28984 49.6885) (width 0.2) (layer "F.Cu") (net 12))
 (segment (start 146.28984 49.6885) (end 150.263468 49.6885) (width 0.2) (layer "F.Cu") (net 12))
 (segment (start 149.80134 37.2) (end 145.573 41.42834) (width 0.2) (layer "F.Cu") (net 12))
 (segment (start 151.834 51.259032) (end 151.834 53.290968) (width 0.2) (layer "F.Cu") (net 12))
 (segment (start 152.094032 53.551) (end 158.000968 53.551) (width 0.2) (layer "F.Cu") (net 12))
 (segment (start 158.000968 53.551) (end 158.93 52.621968) (width 0.2) (layer "F.Cu") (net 12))
 (segment (start 150.263468 49.6885) (end 151.834 51.259032) (width 0.2) (layer "F.Cu") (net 12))
 (segment (start 153.4 37.2) (end 149.80134 37.2) (width 0.2) (layer "F.Cu") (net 12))
 (segment (start 145.573 41.42834) (end 145.573 48.97166) (width 0.2) (layer "F.Cu") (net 12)))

